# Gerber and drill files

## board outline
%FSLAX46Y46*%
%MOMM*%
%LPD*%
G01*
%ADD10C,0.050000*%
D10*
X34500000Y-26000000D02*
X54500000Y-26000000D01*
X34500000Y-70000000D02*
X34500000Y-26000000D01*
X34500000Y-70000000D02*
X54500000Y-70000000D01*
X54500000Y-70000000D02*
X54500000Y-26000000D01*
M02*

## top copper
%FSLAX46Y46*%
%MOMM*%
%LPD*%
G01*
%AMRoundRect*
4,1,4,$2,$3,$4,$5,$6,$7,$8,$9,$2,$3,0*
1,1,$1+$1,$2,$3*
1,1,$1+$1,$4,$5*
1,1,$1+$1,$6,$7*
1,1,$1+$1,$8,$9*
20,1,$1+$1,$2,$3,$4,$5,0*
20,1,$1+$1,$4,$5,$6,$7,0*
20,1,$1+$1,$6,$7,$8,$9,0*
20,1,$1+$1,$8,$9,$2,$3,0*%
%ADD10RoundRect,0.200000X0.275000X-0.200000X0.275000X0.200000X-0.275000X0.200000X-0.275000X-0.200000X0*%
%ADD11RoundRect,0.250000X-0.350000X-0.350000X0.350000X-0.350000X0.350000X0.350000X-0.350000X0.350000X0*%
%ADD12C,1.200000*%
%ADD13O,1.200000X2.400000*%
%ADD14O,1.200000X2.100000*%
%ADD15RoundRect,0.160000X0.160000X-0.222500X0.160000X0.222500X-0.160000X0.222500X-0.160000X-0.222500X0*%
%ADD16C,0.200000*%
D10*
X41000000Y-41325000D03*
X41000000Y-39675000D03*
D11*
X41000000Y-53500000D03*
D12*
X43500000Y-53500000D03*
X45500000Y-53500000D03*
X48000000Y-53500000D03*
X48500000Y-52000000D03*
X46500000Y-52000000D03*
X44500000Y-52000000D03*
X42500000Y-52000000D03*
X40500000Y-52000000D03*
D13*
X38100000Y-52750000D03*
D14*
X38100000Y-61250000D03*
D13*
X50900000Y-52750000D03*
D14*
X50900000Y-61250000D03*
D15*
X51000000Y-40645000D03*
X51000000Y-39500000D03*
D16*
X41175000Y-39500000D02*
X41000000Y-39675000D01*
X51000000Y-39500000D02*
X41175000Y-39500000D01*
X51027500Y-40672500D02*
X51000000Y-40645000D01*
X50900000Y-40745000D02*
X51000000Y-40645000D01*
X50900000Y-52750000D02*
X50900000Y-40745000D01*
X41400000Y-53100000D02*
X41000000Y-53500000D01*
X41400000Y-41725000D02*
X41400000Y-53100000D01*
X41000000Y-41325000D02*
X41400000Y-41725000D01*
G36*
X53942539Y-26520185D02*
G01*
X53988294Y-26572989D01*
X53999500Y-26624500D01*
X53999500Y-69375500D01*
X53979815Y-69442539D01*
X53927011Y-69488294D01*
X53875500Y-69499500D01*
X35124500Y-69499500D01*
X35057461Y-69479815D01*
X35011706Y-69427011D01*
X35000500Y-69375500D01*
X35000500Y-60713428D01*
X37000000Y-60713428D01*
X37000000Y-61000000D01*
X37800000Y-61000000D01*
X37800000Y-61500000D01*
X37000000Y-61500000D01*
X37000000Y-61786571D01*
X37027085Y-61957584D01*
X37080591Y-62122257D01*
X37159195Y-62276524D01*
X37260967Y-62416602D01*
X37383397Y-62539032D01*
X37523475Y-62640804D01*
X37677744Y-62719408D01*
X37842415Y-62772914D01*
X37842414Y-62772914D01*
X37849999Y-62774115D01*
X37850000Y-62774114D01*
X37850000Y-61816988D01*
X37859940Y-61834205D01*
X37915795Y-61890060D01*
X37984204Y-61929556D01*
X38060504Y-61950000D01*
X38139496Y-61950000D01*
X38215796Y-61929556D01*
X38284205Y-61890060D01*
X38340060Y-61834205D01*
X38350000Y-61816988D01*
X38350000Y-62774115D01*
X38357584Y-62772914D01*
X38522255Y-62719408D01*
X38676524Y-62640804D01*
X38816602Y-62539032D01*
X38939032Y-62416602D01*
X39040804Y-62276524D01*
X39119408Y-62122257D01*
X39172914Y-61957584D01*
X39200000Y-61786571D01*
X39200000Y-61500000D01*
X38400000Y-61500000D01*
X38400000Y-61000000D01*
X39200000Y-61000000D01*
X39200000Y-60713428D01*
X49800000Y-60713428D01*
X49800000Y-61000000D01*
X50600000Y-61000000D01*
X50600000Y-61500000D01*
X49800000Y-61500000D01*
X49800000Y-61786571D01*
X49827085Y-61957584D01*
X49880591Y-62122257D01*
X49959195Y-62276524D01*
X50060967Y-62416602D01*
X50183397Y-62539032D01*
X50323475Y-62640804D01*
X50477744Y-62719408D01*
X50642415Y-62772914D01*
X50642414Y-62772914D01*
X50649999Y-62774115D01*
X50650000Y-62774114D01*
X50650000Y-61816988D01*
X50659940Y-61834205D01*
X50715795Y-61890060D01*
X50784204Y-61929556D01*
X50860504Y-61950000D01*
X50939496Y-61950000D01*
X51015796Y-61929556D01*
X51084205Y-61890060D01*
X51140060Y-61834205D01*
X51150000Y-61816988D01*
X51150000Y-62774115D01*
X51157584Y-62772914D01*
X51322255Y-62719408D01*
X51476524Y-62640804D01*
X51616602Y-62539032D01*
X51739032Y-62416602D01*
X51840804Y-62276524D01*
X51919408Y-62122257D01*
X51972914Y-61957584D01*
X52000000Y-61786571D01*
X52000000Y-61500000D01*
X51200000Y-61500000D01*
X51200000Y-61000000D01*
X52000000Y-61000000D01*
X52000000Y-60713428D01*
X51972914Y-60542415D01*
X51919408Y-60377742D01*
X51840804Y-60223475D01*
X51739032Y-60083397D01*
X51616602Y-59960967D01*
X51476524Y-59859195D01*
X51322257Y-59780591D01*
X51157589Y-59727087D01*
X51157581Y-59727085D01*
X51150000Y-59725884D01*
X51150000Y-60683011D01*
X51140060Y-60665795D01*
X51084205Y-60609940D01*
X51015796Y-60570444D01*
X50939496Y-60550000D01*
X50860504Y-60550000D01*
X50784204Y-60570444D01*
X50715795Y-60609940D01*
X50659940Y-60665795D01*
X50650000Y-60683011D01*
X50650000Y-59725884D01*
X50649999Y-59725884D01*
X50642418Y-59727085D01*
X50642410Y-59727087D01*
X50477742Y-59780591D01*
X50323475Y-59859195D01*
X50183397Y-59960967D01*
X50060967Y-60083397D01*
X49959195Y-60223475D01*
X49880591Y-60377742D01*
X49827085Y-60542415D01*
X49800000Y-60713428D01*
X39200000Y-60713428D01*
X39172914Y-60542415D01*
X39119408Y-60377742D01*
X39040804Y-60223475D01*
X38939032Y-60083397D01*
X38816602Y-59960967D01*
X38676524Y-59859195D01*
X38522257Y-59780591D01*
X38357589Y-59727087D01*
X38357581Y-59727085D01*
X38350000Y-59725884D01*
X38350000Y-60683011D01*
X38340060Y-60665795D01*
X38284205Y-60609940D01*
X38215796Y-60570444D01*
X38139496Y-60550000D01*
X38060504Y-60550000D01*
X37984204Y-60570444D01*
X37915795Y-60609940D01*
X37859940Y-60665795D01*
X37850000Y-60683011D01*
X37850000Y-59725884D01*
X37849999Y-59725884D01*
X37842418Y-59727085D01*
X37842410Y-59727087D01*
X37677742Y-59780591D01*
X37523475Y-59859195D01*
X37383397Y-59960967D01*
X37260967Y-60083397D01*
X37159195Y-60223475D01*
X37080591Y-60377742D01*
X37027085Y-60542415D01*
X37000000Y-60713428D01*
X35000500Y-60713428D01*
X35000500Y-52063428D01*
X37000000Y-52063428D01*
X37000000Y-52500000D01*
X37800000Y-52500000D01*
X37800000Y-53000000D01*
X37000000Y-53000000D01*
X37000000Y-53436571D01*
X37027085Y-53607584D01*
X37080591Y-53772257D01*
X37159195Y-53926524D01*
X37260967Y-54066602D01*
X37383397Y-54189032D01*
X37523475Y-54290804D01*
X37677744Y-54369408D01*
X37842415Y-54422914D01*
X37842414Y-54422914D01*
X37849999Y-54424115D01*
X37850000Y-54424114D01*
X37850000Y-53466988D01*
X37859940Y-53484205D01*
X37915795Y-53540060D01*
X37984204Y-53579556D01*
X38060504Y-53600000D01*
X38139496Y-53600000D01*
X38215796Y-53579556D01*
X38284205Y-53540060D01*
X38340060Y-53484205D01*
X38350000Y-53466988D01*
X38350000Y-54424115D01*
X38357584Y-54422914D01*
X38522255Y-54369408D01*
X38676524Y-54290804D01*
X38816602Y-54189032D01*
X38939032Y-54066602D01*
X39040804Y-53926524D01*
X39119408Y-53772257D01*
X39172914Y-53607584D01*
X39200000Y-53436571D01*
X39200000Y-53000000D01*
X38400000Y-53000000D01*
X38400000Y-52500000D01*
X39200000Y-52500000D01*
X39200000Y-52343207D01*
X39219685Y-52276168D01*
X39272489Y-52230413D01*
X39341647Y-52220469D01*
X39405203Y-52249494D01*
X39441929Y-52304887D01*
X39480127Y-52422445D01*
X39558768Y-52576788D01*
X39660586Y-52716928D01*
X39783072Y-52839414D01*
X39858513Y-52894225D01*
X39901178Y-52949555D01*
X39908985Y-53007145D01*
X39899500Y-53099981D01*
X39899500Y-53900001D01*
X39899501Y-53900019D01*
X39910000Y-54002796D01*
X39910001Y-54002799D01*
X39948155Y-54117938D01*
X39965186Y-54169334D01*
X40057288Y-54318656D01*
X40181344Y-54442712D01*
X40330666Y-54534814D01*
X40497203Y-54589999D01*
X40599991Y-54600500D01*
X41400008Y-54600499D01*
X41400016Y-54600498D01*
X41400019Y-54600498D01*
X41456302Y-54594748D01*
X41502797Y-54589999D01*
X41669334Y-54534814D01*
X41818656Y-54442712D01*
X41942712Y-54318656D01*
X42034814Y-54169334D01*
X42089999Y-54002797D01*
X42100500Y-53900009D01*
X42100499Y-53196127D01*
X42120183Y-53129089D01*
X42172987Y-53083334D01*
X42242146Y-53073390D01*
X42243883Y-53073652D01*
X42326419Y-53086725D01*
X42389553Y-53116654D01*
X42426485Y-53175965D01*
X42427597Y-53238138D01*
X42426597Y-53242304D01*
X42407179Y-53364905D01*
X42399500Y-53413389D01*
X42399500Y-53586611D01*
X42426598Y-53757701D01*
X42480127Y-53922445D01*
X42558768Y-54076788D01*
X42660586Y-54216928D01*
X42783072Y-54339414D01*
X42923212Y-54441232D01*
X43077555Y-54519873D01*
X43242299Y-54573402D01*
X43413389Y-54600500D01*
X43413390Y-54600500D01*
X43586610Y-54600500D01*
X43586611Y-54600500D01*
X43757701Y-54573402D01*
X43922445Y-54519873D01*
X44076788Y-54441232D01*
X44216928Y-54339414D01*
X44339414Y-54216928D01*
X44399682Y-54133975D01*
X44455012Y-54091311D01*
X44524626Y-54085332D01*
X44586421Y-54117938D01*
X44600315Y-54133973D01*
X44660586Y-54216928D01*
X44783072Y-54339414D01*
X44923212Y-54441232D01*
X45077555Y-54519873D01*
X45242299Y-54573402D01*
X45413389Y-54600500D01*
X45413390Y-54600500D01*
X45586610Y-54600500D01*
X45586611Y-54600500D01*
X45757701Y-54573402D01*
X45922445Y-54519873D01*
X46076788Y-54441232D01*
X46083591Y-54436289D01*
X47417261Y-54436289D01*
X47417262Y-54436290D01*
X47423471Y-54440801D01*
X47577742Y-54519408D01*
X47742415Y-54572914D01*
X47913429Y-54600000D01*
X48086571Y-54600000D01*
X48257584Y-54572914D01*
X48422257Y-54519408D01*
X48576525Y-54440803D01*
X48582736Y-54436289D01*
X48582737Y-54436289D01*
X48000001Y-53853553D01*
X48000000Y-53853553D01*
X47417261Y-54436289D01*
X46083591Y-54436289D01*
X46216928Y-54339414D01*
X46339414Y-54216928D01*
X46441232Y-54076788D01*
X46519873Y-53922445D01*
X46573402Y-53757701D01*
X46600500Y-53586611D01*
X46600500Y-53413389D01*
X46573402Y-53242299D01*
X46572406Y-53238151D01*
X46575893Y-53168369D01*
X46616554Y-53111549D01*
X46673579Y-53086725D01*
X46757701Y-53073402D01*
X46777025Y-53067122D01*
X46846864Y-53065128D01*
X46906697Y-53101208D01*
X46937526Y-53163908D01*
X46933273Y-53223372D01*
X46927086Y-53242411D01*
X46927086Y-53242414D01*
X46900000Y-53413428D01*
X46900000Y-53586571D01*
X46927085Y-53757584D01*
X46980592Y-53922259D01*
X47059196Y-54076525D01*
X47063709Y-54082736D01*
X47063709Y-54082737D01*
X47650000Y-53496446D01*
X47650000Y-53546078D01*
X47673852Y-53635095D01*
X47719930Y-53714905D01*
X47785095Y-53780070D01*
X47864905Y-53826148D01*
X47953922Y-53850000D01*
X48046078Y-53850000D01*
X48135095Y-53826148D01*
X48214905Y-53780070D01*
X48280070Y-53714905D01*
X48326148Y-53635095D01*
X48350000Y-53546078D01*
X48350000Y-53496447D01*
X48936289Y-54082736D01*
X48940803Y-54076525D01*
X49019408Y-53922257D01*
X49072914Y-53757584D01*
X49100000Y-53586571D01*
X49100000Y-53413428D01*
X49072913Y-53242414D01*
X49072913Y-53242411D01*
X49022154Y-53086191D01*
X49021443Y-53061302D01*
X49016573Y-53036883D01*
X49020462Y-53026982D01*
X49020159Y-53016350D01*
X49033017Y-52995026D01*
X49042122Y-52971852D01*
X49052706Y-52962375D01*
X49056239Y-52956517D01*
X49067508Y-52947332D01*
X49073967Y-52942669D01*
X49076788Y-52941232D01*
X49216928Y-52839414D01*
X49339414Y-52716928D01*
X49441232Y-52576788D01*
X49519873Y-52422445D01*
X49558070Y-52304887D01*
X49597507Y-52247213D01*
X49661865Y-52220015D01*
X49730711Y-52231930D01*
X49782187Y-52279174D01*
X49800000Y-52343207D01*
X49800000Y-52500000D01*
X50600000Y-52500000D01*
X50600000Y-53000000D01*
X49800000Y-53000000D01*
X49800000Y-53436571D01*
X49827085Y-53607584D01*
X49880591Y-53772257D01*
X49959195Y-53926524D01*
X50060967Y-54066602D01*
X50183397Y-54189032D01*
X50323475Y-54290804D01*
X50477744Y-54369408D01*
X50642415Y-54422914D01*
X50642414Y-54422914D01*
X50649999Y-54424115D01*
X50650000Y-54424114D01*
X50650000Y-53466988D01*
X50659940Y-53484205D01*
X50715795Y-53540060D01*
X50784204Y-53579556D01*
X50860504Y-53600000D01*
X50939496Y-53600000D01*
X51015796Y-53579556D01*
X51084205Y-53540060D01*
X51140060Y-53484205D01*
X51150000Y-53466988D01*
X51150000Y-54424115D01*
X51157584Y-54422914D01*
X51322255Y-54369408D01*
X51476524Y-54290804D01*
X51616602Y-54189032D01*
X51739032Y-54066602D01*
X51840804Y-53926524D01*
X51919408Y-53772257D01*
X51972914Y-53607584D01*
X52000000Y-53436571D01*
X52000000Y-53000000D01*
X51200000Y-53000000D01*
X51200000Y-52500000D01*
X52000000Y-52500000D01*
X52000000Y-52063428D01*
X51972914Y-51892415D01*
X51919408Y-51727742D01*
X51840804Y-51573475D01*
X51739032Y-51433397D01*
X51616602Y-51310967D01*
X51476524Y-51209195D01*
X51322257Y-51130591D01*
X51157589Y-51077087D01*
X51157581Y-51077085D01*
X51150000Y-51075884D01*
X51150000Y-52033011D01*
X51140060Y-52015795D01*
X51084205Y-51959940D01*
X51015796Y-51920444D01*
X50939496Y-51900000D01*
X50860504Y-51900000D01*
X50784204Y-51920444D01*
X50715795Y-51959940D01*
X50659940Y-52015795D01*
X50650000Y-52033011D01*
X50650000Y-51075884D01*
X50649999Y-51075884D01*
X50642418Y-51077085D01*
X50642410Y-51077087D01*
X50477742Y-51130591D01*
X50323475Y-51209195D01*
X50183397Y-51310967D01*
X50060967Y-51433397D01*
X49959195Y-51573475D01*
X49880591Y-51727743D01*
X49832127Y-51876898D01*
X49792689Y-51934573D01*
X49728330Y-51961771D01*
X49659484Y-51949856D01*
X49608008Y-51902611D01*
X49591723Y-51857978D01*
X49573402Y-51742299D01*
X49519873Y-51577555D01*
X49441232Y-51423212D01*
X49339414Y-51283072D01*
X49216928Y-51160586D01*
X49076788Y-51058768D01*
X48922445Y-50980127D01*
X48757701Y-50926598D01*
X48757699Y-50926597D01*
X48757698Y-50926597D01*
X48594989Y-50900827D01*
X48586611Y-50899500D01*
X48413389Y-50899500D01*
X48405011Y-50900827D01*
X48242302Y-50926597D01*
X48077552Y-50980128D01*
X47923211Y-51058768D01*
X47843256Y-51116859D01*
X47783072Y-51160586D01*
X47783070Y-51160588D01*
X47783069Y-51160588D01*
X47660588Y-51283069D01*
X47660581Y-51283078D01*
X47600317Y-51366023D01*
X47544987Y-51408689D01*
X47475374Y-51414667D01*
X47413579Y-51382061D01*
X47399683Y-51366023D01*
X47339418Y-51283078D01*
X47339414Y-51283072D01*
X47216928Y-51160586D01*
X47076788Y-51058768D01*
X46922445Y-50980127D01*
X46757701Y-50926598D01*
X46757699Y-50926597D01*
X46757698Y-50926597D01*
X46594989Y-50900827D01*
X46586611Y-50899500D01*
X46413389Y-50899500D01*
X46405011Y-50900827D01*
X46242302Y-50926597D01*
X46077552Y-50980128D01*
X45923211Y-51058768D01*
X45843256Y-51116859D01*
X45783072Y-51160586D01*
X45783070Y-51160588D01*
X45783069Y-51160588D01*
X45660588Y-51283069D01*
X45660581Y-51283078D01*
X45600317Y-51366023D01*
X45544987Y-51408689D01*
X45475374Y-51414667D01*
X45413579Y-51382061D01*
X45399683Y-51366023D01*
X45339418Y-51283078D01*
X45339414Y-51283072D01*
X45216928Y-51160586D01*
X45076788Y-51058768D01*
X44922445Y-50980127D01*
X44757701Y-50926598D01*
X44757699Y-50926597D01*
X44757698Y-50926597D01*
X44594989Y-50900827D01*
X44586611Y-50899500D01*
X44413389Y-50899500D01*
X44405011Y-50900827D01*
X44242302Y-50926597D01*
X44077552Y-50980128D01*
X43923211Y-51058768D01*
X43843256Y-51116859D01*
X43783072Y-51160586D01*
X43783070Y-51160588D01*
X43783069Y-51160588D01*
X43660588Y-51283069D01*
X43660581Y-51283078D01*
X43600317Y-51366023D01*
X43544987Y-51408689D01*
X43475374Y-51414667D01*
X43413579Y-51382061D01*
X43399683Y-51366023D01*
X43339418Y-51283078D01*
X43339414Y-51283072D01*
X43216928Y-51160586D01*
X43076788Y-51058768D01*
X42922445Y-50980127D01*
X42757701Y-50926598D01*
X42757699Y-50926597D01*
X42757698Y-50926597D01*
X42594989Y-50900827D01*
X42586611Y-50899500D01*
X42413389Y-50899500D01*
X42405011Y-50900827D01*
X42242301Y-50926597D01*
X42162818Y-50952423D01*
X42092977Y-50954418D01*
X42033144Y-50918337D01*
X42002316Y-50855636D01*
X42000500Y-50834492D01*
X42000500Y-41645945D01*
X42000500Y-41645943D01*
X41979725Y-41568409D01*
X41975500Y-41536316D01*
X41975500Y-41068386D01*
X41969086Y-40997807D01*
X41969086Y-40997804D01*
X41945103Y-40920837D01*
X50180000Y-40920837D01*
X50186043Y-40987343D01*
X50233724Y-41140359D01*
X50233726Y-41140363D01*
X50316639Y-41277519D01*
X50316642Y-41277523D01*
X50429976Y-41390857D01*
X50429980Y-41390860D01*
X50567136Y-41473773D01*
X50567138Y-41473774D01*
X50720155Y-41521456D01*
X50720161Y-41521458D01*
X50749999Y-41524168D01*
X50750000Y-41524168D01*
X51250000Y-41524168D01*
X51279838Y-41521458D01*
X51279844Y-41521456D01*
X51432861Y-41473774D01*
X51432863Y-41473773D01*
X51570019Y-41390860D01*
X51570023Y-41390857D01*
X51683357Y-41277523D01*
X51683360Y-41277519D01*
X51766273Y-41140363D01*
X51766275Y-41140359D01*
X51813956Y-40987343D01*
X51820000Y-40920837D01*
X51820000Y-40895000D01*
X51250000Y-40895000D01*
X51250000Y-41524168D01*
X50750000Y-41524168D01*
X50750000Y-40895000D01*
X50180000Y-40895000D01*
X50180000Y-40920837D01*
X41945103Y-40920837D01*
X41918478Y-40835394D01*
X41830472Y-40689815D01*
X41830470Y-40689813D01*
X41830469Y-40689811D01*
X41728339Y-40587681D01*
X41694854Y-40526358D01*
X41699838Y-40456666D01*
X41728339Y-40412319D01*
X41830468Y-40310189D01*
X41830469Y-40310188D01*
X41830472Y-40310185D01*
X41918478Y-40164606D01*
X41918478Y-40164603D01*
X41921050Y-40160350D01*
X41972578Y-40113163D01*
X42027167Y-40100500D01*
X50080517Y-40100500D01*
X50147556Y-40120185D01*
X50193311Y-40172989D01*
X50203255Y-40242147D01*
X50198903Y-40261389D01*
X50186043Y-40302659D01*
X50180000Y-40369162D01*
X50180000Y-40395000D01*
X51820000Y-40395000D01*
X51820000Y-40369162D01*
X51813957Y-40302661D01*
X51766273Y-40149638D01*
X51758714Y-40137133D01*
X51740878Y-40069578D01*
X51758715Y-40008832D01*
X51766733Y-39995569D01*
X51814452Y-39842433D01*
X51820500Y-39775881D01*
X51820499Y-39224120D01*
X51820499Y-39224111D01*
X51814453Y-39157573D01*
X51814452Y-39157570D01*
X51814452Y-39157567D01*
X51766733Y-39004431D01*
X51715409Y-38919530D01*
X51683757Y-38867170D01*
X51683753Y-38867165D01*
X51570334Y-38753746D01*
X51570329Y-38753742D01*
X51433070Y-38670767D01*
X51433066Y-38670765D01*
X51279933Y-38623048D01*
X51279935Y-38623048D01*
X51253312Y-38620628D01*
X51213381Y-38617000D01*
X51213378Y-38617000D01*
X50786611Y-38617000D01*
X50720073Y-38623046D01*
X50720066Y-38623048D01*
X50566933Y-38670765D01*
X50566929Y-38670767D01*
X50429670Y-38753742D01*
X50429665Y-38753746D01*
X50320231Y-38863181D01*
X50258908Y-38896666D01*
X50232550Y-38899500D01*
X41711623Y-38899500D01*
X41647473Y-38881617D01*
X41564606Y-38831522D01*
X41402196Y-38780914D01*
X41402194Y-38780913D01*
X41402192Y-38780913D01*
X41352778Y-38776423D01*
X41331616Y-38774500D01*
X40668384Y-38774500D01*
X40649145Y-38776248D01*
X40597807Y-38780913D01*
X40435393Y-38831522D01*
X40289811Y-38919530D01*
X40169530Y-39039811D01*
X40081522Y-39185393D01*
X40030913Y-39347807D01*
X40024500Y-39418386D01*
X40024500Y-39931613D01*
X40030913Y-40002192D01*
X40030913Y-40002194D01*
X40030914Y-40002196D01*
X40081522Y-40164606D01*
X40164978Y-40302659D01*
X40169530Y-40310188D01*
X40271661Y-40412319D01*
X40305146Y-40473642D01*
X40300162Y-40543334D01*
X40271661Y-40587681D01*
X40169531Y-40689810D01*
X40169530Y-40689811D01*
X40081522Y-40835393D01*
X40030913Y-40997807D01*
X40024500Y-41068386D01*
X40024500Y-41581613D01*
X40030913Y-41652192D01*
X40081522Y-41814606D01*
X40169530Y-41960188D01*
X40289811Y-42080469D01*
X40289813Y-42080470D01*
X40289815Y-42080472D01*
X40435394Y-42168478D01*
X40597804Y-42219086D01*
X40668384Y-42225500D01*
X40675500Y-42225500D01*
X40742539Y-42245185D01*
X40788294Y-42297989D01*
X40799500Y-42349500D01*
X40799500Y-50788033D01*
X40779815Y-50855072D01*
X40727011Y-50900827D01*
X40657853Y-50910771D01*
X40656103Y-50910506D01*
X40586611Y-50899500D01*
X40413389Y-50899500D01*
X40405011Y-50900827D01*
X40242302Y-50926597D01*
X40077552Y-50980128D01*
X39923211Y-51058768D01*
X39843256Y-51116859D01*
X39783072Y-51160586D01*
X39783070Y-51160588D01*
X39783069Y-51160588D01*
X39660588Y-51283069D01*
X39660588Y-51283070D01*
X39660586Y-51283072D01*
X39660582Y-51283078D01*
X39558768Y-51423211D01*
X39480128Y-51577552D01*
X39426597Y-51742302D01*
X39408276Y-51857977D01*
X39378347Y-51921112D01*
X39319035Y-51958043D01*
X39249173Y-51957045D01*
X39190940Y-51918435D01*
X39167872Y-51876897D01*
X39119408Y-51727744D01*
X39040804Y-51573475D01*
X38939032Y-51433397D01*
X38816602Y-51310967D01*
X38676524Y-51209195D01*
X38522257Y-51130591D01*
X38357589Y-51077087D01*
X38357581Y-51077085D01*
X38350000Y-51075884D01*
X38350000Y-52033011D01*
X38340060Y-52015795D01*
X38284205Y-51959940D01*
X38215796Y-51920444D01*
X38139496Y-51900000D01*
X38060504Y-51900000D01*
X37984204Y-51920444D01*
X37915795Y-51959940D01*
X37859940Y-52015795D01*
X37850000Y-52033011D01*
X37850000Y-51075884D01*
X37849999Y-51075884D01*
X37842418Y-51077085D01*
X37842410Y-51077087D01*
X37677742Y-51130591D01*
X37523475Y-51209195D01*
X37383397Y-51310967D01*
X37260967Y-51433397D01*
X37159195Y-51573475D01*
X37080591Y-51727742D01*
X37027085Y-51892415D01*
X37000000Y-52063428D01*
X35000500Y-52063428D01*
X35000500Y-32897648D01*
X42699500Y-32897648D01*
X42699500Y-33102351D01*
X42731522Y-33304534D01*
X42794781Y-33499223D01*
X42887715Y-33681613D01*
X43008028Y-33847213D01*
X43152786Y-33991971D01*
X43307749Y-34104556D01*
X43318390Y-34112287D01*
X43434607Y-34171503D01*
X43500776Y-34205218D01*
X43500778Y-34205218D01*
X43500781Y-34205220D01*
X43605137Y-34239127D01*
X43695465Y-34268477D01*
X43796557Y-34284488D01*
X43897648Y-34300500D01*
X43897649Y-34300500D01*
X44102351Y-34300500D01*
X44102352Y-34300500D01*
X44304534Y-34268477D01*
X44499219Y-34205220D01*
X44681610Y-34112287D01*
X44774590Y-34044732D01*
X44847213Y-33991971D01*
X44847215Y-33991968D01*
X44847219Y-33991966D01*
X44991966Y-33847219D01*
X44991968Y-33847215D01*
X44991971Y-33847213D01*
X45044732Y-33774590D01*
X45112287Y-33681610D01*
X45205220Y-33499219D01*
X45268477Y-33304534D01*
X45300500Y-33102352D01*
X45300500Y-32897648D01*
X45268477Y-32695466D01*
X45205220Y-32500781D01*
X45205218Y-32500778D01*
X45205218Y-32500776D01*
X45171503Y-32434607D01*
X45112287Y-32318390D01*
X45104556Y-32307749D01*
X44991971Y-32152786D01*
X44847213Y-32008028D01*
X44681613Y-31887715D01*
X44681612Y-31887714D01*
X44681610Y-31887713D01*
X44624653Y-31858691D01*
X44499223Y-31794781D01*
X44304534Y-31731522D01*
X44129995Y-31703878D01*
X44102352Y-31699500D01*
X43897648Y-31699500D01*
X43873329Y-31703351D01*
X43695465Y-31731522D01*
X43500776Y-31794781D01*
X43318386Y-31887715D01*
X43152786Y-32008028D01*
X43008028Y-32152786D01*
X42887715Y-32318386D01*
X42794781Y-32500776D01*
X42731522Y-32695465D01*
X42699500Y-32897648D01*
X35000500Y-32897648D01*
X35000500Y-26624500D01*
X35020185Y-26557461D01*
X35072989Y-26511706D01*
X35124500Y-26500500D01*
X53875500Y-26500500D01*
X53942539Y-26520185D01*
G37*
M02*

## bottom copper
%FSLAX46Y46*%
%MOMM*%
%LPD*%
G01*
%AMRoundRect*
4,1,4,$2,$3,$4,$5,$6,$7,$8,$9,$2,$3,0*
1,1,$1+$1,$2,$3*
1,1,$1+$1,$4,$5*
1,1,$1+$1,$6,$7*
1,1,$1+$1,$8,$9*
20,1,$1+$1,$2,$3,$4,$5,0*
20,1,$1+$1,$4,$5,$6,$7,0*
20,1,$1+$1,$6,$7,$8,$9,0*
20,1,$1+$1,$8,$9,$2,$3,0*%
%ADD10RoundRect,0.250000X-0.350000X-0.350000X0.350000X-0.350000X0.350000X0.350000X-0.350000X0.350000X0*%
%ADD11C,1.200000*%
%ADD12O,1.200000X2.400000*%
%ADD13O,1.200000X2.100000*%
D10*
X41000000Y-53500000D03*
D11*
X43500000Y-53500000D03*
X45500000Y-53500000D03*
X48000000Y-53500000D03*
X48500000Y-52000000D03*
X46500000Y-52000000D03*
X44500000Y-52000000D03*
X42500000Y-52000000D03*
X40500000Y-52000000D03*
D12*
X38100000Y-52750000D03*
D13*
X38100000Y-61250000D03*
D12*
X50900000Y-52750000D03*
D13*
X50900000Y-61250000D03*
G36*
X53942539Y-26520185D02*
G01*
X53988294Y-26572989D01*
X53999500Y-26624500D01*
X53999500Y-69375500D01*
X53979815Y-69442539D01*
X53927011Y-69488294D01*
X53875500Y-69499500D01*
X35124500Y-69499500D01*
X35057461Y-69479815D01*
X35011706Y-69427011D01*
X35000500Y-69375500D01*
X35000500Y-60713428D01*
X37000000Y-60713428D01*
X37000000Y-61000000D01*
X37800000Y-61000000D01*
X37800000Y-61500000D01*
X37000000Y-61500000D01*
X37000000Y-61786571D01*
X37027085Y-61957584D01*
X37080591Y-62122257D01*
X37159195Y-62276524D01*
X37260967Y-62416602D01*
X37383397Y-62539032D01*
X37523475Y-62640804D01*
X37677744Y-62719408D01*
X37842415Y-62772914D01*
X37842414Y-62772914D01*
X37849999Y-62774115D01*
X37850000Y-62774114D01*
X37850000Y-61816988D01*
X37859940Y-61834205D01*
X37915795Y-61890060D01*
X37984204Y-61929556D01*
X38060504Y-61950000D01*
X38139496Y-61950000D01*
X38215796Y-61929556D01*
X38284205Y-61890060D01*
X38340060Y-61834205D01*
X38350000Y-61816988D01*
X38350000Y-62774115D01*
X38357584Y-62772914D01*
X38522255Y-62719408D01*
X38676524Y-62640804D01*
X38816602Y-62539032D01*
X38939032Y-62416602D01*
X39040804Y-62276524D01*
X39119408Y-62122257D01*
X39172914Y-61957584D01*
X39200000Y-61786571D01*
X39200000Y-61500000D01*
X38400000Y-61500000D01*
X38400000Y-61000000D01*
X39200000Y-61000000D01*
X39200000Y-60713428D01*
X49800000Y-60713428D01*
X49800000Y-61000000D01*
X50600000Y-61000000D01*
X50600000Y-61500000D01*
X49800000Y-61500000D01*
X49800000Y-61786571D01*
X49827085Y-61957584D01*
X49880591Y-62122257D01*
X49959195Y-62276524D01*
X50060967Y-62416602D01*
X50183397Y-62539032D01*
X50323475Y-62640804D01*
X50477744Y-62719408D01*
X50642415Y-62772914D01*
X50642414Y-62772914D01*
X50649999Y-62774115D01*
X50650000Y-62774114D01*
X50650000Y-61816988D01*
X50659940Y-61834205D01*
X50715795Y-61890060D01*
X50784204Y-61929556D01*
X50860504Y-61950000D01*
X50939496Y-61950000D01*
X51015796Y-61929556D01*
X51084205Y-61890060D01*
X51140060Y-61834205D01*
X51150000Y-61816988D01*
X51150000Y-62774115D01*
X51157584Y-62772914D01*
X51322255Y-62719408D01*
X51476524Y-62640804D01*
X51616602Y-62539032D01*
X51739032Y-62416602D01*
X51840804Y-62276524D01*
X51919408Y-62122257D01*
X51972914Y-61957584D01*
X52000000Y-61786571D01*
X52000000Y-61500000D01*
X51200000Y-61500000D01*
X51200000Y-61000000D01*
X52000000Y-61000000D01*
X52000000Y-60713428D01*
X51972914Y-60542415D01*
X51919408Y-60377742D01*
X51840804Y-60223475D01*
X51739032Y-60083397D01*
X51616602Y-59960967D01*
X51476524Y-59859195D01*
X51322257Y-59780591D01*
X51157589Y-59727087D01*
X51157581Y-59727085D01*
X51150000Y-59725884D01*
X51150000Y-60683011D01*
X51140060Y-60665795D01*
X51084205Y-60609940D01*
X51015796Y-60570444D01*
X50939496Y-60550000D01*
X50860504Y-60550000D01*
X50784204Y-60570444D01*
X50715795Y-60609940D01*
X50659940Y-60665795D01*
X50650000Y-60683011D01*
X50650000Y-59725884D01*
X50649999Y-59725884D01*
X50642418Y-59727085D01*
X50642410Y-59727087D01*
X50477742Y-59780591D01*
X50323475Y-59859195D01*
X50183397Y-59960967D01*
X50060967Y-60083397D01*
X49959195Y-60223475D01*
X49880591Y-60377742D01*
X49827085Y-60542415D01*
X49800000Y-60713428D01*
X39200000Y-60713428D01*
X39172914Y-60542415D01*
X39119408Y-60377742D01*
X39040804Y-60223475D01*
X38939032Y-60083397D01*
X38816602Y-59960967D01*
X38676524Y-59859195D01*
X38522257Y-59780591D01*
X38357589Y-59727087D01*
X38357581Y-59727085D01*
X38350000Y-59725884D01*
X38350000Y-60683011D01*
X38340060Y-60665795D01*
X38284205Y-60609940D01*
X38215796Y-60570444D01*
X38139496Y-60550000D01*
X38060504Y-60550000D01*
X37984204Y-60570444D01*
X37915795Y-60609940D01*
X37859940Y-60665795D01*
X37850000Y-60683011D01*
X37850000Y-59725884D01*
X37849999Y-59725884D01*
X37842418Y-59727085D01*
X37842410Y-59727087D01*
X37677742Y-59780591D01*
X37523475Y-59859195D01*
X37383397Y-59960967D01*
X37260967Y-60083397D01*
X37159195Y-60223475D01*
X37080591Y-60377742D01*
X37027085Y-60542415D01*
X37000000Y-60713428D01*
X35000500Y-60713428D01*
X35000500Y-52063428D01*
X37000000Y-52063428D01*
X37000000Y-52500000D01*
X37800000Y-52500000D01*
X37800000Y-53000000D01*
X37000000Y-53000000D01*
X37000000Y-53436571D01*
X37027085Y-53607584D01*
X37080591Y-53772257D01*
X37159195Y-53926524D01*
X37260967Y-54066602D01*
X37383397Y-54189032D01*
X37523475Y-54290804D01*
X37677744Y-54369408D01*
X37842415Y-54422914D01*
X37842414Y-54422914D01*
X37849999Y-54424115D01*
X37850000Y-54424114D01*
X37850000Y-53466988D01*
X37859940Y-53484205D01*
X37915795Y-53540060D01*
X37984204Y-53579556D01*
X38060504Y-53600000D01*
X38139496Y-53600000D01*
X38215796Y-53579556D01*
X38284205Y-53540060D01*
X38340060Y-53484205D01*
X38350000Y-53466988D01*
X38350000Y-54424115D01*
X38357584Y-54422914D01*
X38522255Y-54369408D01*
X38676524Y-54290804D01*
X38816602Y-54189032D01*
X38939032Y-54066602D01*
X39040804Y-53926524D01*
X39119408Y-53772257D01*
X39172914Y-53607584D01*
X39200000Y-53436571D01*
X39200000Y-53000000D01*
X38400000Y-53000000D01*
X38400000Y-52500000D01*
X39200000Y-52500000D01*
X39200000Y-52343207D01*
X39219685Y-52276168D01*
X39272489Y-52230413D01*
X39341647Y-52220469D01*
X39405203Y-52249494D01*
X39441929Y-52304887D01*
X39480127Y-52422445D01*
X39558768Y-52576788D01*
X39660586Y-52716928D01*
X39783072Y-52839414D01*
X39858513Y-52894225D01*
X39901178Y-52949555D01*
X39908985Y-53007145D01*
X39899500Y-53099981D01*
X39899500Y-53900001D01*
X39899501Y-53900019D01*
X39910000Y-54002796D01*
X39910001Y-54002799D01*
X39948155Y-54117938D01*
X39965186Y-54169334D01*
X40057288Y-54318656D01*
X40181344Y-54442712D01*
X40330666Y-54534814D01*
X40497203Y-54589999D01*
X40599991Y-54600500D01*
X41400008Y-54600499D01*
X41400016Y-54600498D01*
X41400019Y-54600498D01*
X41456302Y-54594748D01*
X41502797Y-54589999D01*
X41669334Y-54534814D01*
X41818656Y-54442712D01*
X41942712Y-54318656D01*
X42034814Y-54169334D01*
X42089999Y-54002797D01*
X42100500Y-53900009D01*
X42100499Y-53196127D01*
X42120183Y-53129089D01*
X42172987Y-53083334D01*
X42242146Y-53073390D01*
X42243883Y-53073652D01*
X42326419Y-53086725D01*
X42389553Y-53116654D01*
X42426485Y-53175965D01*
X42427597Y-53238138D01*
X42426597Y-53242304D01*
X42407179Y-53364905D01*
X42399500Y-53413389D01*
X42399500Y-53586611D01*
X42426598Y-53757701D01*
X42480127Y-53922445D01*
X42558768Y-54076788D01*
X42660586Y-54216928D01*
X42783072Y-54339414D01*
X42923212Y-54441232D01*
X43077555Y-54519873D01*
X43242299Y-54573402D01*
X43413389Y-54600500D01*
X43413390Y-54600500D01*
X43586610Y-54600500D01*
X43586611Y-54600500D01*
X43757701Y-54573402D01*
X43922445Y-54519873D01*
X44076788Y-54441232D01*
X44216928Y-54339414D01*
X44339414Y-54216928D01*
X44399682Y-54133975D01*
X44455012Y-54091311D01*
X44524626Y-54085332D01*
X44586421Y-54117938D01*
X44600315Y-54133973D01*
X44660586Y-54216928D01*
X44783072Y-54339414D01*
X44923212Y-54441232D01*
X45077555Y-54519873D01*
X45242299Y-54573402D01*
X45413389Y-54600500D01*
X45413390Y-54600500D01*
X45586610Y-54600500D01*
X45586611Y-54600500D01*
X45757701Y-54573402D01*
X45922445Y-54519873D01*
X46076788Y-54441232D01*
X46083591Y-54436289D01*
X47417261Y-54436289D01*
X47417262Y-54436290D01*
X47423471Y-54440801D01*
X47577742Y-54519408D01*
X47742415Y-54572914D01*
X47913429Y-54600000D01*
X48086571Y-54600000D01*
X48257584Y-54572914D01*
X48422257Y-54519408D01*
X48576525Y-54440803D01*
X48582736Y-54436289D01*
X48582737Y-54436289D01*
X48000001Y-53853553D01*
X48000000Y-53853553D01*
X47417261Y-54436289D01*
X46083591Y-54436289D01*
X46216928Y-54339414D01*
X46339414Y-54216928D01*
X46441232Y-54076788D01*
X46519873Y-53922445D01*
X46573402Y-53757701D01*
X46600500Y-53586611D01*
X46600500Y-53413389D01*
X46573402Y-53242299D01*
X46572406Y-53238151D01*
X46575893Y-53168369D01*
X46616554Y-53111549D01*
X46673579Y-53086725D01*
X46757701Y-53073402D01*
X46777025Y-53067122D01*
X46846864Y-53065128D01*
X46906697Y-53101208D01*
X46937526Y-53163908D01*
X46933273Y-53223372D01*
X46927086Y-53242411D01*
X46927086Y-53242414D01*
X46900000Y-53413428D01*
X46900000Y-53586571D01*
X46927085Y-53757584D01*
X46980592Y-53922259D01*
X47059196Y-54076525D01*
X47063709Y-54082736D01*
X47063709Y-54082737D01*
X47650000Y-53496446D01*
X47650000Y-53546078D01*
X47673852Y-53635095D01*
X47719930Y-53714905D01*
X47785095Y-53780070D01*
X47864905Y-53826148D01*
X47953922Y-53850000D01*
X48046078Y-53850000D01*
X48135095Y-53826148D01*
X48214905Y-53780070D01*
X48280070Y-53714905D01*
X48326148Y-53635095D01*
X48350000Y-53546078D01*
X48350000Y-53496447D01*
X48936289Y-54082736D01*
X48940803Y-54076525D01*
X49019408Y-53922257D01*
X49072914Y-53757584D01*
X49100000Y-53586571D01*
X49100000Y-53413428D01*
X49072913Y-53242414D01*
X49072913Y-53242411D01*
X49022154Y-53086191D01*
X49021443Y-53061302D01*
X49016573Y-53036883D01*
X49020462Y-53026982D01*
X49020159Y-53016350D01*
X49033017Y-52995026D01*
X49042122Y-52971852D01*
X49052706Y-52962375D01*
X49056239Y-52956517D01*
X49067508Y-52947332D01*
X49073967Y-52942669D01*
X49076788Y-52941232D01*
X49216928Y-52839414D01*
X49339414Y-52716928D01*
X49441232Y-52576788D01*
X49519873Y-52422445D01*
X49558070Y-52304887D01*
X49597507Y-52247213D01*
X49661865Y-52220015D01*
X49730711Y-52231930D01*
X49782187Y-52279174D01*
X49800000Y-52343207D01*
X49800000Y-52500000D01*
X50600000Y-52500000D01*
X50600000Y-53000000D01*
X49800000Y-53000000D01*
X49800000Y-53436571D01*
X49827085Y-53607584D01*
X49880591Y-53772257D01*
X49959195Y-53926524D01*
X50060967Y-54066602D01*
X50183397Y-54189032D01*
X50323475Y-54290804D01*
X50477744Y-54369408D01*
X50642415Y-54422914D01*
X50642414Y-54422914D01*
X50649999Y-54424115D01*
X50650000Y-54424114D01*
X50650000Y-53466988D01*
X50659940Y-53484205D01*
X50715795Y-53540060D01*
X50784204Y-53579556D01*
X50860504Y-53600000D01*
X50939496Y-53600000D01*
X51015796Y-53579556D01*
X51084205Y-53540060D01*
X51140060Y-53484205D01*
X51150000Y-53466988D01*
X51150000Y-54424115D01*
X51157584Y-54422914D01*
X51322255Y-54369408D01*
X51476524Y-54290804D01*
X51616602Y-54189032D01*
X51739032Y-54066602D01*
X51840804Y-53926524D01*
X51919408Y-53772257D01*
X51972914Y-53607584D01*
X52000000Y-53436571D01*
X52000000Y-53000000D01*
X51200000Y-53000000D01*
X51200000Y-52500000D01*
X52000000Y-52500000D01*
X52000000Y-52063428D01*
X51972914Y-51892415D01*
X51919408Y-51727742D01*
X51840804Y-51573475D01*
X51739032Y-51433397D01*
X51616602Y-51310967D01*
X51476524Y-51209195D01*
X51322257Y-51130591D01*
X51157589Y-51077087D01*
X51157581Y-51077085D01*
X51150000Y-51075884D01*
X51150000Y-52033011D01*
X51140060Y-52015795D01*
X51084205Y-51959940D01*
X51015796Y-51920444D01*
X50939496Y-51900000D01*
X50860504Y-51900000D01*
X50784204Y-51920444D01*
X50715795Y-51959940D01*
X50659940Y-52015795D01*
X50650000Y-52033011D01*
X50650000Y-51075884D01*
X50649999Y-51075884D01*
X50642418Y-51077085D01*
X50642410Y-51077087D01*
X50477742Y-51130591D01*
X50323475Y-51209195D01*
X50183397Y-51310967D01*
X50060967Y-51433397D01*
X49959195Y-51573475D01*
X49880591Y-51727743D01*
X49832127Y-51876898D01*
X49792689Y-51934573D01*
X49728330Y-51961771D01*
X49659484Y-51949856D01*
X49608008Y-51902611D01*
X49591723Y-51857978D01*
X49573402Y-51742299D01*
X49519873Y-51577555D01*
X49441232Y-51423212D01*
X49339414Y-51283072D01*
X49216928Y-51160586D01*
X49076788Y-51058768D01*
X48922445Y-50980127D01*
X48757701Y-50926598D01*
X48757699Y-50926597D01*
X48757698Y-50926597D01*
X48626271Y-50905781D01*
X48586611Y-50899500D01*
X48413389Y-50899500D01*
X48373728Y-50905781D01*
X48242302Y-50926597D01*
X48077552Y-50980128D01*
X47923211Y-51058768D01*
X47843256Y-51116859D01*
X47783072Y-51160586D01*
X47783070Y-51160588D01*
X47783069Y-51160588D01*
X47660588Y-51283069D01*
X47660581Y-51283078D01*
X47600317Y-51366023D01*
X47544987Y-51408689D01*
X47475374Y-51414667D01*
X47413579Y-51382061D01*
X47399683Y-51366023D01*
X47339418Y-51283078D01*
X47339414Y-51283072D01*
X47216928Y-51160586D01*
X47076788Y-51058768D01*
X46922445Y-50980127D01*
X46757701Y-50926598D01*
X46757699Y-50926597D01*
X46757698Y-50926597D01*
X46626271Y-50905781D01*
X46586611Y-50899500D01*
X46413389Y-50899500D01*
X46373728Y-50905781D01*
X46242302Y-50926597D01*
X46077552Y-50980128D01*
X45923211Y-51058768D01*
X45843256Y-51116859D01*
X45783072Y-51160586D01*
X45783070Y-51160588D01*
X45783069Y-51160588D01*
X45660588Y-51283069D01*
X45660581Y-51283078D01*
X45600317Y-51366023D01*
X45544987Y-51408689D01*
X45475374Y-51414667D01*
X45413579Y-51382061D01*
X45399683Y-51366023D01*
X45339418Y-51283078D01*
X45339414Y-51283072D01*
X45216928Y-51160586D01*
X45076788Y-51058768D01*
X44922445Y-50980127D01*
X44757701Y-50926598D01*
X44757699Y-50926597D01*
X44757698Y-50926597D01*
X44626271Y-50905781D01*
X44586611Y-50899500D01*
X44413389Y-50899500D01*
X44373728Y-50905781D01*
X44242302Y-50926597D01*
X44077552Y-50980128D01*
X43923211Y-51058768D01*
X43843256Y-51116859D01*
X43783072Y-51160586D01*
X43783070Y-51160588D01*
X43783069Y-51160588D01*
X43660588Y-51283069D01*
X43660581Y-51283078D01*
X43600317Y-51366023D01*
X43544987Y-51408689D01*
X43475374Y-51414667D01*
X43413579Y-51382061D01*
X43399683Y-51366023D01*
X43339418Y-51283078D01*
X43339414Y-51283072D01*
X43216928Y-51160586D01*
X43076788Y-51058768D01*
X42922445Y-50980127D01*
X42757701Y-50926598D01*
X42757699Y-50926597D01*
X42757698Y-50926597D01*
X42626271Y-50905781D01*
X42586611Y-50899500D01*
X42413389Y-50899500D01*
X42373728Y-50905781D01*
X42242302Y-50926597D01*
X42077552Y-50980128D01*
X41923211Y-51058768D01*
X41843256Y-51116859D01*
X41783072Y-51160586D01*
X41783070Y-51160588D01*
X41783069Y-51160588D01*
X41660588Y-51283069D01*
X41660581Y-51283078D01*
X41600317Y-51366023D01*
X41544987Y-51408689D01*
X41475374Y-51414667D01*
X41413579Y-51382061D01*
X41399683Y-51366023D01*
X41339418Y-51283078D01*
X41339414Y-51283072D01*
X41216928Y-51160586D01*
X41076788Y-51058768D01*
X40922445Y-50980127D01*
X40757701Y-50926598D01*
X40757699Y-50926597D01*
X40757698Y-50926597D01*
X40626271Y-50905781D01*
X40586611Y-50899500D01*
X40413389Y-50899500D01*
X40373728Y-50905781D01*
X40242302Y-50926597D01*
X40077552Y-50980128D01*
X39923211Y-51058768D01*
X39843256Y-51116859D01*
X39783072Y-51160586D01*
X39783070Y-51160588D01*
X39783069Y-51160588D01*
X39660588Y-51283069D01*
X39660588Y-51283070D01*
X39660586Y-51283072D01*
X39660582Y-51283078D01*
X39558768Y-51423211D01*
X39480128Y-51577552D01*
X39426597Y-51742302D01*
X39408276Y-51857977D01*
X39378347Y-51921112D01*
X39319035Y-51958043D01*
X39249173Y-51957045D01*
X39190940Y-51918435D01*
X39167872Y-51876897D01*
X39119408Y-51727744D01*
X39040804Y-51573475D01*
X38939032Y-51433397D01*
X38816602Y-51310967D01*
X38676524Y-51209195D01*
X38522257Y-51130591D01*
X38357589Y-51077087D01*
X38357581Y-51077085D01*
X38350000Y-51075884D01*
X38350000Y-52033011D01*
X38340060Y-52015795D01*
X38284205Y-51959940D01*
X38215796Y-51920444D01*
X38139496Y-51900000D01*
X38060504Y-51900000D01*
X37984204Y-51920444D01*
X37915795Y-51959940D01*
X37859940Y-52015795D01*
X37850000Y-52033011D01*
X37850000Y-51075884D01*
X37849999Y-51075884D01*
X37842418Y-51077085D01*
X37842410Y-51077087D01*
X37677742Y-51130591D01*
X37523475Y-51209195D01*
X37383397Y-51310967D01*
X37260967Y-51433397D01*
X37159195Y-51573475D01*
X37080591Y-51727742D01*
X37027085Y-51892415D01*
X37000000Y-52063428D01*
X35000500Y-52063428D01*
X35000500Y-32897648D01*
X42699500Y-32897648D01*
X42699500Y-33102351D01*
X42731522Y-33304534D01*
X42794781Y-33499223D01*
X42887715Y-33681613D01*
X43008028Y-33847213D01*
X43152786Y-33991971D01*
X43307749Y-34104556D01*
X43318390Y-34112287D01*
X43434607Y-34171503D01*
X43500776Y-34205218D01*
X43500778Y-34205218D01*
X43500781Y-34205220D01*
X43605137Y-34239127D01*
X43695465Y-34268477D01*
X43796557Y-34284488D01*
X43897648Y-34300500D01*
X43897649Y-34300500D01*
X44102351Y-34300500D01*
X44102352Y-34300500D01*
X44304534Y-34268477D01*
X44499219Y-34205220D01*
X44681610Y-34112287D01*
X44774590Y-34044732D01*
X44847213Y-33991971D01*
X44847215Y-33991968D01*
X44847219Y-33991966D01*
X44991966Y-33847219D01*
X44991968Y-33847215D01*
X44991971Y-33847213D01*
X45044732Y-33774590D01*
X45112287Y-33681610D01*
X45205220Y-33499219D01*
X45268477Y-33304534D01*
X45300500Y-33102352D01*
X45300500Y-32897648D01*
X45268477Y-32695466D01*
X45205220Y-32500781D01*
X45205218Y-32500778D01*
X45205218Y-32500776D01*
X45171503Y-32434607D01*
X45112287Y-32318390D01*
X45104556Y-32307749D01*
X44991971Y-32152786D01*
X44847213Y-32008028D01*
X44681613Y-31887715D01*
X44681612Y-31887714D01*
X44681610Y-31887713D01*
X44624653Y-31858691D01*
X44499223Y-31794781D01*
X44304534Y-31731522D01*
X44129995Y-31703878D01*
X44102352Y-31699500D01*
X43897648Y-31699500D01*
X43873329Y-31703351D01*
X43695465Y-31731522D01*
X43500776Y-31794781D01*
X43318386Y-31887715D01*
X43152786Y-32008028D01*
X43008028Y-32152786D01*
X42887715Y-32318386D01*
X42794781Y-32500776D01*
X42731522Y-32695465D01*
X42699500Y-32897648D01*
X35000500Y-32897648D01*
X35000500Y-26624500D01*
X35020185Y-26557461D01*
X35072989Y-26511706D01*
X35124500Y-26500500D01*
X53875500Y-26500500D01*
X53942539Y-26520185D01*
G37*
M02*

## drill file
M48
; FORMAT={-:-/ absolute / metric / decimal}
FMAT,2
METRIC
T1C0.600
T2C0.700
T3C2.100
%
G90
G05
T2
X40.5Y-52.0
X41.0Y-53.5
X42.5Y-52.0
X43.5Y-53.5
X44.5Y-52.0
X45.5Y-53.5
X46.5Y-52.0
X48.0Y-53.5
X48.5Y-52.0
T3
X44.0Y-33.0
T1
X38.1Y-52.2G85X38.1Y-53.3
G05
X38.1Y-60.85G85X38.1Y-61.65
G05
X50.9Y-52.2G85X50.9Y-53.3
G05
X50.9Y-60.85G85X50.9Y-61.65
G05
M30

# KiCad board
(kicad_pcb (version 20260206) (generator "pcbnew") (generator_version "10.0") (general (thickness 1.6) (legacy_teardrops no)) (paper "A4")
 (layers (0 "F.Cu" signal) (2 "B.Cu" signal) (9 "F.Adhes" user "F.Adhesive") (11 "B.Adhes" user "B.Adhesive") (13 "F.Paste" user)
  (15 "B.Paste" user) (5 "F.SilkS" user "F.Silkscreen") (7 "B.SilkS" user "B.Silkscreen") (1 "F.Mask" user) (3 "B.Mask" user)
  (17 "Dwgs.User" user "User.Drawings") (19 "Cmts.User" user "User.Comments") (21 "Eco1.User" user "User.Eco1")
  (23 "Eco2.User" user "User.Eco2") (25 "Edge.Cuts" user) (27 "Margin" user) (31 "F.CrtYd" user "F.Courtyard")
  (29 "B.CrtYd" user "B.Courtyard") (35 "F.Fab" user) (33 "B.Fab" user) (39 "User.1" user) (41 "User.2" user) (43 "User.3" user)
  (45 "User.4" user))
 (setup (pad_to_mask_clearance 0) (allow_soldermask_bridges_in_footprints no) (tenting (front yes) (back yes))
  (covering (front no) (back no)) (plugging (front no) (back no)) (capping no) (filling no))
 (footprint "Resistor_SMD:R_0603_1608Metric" (layer "F.Cu") (at 41 40.5 90)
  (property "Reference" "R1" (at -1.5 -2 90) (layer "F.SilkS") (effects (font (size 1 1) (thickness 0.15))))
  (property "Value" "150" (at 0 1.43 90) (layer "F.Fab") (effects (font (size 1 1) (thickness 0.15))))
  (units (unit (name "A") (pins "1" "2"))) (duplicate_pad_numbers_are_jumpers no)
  (pad "1" smd roundrect (at -0.825 0 90) (size 0.8 0.95) (layers "F.Cu" "F.Mask" "F.Paste") (roundrect_rratio 0.25)
   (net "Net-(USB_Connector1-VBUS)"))
  (pad "2" smd roundrect (at 0.825 0 90) (size 0.8 0.95) (layers "F.Cu" "F.Mask" "F.Paste") (roundrect_rratio 0.25) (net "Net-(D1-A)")))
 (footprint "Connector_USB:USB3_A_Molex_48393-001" (layer "F.Cu") (at 41 53.5)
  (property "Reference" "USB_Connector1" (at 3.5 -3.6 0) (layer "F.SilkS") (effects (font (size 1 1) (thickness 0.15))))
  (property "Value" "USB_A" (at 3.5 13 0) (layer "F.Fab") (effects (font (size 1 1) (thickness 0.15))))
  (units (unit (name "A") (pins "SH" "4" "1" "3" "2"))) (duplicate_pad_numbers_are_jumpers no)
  (pad "1" thru_hole roundrect (at 0 0) (size 1.2 1.2) (drill 0.7) (layers "*.Cu" "*.Mask") (remove_unused_layers no)
   (roundrect_rratio 0.2083333333) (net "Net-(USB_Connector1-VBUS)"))
  (pad "2" thru_hole circle (at 2.5 0) (size 1.2 1.2) (drill 0.7) (layers "*.Cu" "*.Mask") (remove_unused_layers no)
   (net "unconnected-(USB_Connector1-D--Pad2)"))
  (pad "3" thru_hole circle (at 4.5 0) (size 1.2 1.2) (drill 0.7) (layers "*.Cu" "*.Mask") (remove_unused_layers no)
   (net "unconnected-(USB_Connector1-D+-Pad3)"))
  (pad "4" thru_hole circle (at 7 0) (size 1.2 1.2) (drill 0.7) (layers "*.Cu" "*.Mask") (remove_unused_layers no) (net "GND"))
  (pad "5" thru_hole circle (at 7.5 -1.5) (size 1.2 1.2) (drill 0.7) (layers "*.Cu" "*.Mask") (remove_unused_layers no))
  (pad "6" thru_hole circle (at 5.5 -1.5) (size 1.2 1.2) (drill 0.7) (layers "*.Cu" "*.Mask") (remove_unused_layers no))
  (pad "7" thru_hole circle (at 3.5 -1.5) (size 1.2 1.2) (drill 0.7) (layers "*.Cu" "*.Mask") (remove_unused_layers no))
  (pad "8" thru_hole circle (at 1.5 -1.5) (size 1.2 1.2) (drill 0.7) (layers "*.Cu" "*.Mask") (remove_unused_layers no))
  (pad "9" thru_hole circle (at -0.5 -1.5) (size 1.2 1.2) (drill 0.7) (layers "*.Cu" "*.Mask") (remove_unused_layers no))
  (pad "SH" thru_hole oval (at -2.9 -0.75) (size 1.2 2.4) (drill oval 0.6 1.7) (layers "*.Cu" "*.Mask") (remove_unused_layers no)
   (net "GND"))
  (pad "SH" thru_hole oval (at -2.9 7.75) (size 1.2 2.1) (drill oval 0.6 1.4) (layers "*.Cu" "*.Mask") (remove_unused_layers no) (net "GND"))
  (pad "SH" thru_hole oval (at 9.9 -0.75) (size 1.2 2.4) (drill oval 0.6 1.7) (layers "*.Cu" "*.Mask") (remove_unused_layers no) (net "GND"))
  (pad "SH" thru_hole oval (at 9.9 7.75) (size 1.2 2.1) (drill oval 0.6 1.4) (layers "*.Cu" "*.Mask") (remove_unused_layers no) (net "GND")))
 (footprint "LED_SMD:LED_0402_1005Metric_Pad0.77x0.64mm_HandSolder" (layer "F.Cu") (at 51 40.0725 90)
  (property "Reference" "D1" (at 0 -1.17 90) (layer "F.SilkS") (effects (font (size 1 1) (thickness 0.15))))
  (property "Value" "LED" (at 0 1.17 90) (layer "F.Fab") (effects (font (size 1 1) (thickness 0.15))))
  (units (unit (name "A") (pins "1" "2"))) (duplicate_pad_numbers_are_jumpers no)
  (pad "1" smd roundrect (at -0.5725 0 90) (size 0.765 0.64) (layers "F.Cu" "F.Mask" "F.Paste") (roundrect_rratio 0.25) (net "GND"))
  (pad "2" smd roundrect (at 0.5725 0 90) (size 0.765 0.64) (layers "F.Cu" "F.Mask" "F.Paste") (roundrect_rratio 0.25) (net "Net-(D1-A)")))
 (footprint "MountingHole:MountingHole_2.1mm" (layer "F.Cu") (at 44 33)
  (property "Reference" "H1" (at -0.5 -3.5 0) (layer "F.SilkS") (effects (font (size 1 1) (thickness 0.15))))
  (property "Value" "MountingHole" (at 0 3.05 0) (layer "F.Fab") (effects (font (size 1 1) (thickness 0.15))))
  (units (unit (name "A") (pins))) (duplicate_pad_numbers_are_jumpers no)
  (pad "" np_thru_hole circle (at 0 0) (size 2.1 2.1) (drill 2.1) (layers "*.Cu" "*.Mask")))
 (gr_line (start 34.5 26) (end 54.5 26) (stroke (width 0.05) (type default)) (layer "Edge.Cuts"))
 (gr_line (start 34.5 70) (end 34.5 26) (stroke (width 0.05) (type default)) (layer "Edge.Cuts"))
 (gr_line (start 34.5 70) (end 54.5 70) (stroke (width 0.05) (type default)) (layer "Edge.Cuts"))
 (gr_line (start 54.5 70) (end 54.5 26) (stroke (width 0.05) (type default)) (layer "Edge.Cuts"))
 (segment (start 41.175 39.5) (end 41 39.675) (width 0.2) (layer "F.Cu") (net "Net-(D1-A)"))
 (segment (start 51 39.5) (end 41.175 39.5) (width 0.2) (layer "F.Cu") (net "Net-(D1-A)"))
 (segment (start 51.0275 40.6725) (end 51 40.645) (width 0.2) (layer "F.Cu") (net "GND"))
 (segment (start 50.9 40.745) (end 51 40.645) (width 0.2) (layer "F.Cu") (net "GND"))
 (segment (start 50.9 52.75) (end 50.9 40.745) (width 0.2) (layer "F.Cu") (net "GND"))
 (segment (start 41.4 53.1) (end 41 53.5) (width 0.2) (layer "F.Cu") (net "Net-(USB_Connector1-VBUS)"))
 (segment (start 41.4 41.725) (end 41.4 53.1) (width 0.2) (layer "F.Cu") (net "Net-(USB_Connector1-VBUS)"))
 (segment (start 41 41.325) (end 41.4 41.725) (width 0.2) (layer "F.Cu") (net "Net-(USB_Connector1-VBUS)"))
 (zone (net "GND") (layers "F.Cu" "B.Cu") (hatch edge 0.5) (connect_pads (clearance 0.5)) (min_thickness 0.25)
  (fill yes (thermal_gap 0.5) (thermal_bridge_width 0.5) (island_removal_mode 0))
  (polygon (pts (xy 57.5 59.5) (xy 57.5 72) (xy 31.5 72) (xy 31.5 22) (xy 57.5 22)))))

